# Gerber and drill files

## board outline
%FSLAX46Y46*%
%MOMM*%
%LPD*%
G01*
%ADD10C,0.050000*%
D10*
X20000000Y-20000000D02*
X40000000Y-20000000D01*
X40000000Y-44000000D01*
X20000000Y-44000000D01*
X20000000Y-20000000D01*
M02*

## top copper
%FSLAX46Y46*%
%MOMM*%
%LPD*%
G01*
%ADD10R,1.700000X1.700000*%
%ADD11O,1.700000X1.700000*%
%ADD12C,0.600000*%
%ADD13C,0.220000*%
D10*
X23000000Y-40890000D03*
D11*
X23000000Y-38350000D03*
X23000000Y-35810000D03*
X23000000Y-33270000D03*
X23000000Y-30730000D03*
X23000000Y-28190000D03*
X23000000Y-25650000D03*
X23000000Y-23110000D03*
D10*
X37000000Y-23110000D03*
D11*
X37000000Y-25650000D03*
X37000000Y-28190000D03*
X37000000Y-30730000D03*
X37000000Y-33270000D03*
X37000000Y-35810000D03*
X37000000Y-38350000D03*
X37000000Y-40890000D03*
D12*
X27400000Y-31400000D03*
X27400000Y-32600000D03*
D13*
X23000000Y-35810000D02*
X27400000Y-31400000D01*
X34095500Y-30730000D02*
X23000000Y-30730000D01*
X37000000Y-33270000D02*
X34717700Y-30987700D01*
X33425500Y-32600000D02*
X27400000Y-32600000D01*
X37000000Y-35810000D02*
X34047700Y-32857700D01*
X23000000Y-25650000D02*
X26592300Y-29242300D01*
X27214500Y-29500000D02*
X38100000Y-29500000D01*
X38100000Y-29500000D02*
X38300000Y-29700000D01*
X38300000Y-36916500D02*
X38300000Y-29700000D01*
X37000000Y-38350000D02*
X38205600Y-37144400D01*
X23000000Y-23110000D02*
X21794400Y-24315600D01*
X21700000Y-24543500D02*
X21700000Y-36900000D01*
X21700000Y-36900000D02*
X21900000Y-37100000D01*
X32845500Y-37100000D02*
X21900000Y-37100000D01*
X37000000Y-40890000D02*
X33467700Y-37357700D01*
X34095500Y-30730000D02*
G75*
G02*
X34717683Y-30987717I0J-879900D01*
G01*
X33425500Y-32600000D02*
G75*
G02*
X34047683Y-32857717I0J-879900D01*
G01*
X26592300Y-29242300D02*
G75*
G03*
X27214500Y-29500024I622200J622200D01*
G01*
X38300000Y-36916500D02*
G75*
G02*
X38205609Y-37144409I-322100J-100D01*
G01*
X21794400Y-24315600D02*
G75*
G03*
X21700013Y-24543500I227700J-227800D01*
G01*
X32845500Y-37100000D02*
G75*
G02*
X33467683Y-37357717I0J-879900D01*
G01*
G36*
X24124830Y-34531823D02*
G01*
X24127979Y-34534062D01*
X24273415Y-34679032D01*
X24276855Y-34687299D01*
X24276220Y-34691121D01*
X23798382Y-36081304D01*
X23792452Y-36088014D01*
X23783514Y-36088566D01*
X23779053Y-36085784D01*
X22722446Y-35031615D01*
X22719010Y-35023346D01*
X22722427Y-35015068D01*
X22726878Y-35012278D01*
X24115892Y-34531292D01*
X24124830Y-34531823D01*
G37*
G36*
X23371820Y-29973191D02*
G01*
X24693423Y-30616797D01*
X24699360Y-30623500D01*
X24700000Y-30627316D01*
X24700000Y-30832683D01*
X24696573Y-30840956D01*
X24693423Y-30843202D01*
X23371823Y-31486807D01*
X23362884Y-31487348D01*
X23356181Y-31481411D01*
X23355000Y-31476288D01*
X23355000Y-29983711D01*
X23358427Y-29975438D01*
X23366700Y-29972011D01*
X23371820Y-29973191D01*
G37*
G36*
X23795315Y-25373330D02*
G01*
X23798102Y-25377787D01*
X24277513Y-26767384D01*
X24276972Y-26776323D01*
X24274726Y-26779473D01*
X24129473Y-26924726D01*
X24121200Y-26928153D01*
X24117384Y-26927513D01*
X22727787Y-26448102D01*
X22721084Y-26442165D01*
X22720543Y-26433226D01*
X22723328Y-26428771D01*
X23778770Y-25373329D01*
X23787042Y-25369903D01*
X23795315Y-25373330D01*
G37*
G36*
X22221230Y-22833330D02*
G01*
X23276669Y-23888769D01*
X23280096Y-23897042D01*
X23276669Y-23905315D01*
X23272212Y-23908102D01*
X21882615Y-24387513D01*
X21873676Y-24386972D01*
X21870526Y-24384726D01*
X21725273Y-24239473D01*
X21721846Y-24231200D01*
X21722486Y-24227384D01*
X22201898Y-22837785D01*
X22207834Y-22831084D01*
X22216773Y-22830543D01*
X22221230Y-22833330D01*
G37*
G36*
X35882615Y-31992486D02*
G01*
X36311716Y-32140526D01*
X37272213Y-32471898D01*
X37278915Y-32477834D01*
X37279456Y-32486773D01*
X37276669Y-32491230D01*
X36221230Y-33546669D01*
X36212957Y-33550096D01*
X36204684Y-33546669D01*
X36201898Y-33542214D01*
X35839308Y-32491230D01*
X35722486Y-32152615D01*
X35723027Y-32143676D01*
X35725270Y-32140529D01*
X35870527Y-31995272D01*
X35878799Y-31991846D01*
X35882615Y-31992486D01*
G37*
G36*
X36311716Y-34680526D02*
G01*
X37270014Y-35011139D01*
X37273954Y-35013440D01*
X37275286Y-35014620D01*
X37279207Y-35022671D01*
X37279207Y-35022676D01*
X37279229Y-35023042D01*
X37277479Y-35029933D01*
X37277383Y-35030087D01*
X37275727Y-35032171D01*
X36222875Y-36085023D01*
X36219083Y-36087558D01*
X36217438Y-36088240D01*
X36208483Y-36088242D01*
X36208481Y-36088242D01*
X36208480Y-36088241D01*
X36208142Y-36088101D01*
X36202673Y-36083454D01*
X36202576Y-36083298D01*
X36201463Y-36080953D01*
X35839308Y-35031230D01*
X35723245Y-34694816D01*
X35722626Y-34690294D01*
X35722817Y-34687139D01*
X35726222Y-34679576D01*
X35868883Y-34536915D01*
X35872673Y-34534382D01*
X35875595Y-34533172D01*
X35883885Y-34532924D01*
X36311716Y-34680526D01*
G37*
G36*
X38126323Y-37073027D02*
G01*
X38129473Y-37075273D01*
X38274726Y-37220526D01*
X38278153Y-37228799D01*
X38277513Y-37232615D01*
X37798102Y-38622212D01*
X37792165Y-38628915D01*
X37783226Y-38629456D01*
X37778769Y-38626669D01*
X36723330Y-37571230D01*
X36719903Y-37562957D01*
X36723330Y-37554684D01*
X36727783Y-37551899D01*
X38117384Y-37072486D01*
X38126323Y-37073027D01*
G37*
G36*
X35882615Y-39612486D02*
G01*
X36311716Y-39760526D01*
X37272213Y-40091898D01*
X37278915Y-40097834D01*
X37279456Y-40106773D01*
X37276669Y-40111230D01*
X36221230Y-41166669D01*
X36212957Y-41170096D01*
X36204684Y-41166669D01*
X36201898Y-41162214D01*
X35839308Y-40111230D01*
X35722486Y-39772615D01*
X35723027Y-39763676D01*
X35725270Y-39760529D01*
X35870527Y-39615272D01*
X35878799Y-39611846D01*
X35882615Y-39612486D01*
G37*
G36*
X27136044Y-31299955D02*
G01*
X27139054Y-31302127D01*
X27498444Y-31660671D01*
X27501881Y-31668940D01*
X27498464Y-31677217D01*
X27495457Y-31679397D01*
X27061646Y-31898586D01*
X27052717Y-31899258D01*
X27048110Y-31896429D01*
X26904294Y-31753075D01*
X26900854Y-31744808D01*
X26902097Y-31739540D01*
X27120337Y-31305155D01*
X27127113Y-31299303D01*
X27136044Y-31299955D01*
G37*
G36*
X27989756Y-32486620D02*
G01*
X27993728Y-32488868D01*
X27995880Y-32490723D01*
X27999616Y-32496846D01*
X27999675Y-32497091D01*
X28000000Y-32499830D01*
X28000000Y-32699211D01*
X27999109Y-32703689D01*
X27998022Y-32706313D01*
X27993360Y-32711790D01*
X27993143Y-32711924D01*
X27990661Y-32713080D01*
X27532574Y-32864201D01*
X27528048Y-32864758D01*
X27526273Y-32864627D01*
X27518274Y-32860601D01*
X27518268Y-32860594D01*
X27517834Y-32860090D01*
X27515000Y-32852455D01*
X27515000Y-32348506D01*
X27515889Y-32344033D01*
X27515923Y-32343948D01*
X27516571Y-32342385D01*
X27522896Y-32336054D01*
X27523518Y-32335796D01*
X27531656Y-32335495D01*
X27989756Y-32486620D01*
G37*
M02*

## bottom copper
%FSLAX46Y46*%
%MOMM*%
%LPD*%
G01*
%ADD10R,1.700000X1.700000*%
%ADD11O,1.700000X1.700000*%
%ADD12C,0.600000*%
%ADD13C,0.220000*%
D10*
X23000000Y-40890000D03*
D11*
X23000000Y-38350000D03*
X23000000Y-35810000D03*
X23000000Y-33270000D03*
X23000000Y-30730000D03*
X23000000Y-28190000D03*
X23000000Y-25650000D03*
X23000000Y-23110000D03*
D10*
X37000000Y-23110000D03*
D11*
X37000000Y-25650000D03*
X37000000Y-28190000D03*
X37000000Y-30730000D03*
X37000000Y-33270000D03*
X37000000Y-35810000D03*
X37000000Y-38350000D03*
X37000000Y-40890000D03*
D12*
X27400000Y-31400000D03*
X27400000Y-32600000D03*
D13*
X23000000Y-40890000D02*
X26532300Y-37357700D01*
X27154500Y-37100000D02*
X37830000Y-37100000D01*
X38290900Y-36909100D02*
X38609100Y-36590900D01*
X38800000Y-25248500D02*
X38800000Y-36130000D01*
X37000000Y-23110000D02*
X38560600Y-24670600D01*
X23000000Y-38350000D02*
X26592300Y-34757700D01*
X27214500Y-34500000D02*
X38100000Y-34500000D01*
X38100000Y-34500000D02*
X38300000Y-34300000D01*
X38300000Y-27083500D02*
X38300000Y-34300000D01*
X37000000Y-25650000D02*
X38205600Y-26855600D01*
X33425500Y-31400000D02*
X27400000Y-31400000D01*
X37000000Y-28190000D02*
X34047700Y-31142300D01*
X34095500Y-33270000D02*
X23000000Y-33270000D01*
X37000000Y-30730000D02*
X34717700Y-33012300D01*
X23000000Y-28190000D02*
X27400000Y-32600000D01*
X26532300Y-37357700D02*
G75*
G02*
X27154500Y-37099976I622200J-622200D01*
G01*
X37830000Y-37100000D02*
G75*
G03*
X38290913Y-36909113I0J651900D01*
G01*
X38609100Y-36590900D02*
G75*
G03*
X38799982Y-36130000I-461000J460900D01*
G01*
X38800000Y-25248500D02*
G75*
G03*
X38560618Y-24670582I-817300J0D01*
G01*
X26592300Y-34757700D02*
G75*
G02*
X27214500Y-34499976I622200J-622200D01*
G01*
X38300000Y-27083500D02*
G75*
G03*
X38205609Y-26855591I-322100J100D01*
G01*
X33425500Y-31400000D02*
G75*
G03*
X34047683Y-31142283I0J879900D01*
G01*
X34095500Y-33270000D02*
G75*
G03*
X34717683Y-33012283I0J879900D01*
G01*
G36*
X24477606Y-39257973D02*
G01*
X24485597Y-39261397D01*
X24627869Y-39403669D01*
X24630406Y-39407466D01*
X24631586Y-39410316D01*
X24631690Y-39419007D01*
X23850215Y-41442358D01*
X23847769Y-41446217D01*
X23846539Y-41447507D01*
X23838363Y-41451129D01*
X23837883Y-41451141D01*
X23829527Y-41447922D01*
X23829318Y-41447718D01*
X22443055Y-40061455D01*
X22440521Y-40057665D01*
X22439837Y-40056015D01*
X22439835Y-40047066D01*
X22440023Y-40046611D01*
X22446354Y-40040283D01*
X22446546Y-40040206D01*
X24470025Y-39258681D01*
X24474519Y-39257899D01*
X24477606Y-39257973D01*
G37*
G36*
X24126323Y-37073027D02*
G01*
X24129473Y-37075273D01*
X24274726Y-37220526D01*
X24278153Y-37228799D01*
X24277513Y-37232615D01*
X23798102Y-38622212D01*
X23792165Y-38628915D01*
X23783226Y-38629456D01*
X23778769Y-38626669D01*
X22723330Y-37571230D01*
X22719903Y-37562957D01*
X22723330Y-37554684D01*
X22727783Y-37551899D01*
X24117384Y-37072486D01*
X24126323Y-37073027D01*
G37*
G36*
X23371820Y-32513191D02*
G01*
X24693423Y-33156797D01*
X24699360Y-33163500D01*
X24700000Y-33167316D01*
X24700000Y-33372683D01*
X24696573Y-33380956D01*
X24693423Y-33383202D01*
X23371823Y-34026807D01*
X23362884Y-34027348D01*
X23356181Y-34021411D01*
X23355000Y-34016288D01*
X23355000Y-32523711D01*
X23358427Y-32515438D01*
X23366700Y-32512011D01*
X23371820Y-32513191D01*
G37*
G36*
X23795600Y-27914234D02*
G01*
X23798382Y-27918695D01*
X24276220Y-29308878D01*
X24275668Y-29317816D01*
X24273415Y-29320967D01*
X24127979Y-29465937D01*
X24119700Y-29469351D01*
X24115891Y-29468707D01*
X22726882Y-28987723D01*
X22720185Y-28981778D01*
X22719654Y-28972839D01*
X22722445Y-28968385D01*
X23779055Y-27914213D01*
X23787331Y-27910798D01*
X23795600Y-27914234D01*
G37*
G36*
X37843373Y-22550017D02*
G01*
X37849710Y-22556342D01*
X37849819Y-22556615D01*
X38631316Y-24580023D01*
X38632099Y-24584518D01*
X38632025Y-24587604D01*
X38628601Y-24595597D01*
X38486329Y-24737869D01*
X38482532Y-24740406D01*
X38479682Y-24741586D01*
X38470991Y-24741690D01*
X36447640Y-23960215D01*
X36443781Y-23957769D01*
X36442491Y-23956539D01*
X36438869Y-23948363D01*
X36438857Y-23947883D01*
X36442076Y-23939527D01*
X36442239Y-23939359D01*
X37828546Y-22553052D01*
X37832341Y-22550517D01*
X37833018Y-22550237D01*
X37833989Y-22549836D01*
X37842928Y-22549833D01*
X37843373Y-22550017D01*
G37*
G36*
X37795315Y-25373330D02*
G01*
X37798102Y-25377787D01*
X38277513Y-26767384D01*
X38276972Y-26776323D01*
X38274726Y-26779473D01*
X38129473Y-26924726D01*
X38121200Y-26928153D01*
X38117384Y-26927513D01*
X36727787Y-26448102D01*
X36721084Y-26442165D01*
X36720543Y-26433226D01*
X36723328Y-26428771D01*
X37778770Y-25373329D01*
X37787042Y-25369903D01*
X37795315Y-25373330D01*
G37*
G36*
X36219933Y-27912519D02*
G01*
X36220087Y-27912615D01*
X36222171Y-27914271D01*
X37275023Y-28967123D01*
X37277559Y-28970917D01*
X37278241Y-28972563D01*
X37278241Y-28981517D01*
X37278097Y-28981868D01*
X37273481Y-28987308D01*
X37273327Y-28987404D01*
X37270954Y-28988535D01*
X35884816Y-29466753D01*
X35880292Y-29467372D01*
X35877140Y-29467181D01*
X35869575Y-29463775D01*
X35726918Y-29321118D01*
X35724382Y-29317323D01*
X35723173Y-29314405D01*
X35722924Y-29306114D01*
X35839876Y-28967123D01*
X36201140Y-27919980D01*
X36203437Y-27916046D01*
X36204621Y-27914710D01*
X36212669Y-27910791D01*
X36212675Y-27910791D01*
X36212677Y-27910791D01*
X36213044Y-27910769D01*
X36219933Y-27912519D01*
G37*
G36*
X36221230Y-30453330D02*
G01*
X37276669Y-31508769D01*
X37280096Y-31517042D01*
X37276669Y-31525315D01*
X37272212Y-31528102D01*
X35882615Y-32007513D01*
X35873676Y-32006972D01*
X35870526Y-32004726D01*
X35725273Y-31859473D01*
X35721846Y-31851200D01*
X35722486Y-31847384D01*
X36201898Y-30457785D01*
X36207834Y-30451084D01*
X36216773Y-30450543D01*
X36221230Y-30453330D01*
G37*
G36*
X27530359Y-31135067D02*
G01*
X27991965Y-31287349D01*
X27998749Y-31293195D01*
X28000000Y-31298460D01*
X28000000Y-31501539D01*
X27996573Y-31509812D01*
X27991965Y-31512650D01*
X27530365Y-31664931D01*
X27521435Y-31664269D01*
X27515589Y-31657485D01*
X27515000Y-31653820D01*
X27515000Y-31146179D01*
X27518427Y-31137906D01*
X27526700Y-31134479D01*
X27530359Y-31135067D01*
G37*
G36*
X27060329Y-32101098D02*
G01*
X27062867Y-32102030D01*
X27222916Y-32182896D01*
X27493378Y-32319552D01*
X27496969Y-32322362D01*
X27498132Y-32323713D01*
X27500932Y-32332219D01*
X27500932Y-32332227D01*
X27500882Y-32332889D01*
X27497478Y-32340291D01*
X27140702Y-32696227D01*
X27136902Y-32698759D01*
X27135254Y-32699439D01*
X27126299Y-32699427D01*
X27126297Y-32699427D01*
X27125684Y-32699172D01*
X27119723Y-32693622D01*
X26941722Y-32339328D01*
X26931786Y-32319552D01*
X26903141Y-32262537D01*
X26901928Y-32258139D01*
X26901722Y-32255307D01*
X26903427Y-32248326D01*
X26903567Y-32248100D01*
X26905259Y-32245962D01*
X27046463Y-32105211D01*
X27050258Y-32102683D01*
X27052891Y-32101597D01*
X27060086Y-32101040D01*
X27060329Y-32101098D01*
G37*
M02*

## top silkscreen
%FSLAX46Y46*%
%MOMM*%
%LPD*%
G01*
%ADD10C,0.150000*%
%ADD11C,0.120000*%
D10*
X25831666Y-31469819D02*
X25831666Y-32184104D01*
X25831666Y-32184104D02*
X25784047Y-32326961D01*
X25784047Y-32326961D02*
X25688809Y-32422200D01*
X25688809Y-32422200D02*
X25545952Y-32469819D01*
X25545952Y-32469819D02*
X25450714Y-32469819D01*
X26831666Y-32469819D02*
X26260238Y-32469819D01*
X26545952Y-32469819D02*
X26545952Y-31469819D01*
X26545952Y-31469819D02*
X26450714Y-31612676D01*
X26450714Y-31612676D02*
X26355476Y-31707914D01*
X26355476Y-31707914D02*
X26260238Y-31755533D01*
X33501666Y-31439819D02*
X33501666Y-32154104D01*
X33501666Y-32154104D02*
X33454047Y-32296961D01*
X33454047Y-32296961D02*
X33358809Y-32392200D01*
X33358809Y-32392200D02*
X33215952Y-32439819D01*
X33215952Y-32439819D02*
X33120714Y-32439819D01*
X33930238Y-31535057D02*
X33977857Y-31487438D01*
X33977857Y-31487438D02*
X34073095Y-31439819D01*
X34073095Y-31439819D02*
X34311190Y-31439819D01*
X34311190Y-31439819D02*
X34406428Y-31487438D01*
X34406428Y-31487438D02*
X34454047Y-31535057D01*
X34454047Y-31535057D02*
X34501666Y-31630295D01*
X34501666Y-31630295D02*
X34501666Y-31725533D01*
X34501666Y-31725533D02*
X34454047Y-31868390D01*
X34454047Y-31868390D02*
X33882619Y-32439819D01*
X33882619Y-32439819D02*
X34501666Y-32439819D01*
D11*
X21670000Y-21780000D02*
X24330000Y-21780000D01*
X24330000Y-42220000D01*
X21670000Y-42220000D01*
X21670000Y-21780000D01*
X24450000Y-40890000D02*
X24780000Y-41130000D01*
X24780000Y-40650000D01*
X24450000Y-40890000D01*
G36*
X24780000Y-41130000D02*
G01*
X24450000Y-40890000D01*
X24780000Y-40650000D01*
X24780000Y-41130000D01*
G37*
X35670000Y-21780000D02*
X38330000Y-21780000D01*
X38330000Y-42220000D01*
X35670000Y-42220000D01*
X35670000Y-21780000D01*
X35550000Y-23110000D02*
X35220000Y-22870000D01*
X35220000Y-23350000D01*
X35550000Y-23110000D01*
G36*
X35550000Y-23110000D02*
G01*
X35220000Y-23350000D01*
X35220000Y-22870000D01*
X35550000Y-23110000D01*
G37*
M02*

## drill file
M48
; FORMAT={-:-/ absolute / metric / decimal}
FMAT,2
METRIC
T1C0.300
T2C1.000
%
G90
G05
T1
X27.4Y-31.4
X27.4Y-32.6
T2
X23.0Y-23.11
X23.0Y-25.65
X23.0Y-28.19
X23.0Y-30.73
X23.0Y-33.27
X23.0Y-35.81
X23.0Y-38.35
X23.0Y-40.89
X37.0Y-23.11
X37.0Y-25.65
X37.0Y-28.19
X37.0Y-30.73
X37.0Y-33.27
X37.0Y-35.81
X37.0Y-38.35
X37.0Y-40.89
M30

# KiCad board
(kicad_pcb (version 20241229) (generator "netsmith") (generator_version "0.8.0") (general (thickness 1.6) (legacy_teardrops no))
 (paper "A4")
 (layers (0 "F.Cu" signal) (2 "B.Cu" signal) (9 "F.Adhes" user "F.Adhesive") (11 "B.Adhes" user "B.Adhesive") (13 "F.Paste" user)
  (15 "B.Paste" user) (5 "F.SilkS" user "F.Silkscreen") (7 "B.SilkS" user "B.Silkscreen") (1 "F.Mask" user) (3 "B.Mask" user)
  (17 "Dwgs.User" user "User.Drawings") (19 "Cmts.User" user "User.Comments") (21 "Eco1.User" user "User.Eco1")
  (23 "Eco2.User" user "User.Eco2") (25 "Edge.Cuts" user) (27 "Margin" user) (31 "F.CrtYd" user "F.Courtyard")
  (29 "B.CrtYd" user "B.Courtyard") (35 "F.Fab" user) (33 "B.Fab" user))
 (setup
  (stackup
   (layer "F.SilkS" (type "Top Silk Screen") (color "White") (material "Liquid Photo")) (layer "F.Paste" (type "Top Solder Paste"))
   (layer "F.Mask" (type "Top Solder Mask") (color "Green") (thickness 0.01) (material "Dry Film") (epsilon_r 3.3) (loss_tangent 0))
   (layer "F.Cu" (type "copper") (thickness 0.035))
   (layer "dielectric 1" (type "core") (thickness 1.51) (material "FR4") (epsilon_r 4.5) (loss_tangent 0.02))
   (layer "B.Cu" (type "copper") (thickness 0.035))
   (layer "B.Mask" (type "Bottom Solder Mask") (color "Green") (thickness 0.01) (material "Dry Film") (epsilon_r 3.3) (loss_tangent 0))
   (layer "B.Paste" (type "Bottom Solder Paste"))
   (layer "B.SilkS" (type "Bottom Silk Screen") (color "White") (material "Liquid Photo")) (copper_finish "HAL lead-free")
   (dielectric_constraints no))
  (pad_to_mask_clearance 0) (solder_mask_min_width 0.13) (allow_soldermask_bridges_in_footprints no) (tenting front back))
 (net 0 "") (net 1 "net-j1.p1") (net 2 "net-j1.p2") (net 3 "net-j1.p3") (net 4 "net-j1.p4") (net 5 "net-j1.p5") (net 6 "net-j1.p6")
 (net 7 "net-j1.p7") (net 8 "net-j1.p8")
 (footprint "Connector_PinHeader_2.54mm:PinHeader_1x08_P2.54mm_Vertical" (layer "F.Cu") (at 23 40.89 180)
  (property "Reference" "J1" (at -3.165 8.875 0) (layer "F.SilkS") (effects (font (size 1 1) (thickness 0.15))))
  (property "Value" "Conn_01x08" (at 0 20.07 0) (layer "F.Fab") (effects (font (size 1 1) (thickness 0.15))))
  (pad "1" thru_hole rect (at 0 0 180) (size 1.7 1.7) (drill 1) (layers "*.Cu" "*.Mask") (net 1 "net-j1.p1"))
  (pad "2" thru_hole oval (at 0 2.54 180) (size 1.7 1.7) (drill 1) (layers "*.Cu" "*.Mask") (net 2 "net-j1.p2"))
  (pad "3" thru_hole oval (at 0 5.08 180) (size 1.7 1.7) (drill 1) (layers "*.Cu" "*.Mask") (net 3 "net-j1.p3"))
  (pad "4" thru_hole oval (at 0 7.62 180) (size 1.7 1.7) (drill 1) (layers "*.Cu" "*.Mask") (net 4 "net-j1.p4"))
  (pad "5" thru_hole oval (at 0 10.16 180) (size 1.7 1.7) (drill 1) (layers "*.Cu" "*.Mask") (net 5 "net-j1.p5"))
  (pad "6" thru_hole oval (at 0 12.7 180) (size 1.7 1.7) (drill 1) (layers "*.Cu" "*.Mask") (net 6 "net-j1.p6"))
  (pad "7" thru_hole oval (at 0 15.24 180) (size 1.7 1.7) (drill 1) (layers "*.Cu" "*.Mask") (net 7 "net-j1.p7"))
  (pad "8" thru_hole oval (at 0 17.78 180) (size 1.7 1.7) (drill 1) (layers "*.Cu" "*.Mask") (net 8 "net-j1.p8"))
  (fp_rect (start -1.33 -1.33) (end 1.33 19.11) (stroke (width 0.12) (type solid)) (fill no) (layer "F.SilkS"))
  (fp_poly (pts (xy -1.45 0) (xy -1.78 -0.24) (xy -1.78 0.24)) (stroke (width 0.12) (type solid)) (fill solid) (layer "F.SilkS")))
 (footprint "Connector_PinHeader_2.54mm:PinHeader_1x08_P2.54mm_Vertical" (layer "F.Cu") (at 37 23.11)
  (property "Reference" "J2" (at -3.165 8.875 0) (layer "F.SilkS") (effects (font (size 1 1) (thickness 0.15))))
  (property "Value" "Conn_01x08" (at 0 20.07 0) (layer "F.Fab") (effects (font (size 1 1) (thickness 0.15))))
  (pad "1" thru_hole rect (at 0 0) (size 1.7 1.7) (drill 1) (layers "*.Cu" "*.Mask") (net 1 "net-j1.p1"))
  (pad "2" thru_hole oval (at 0 2.54) (size 1.7 1.7) (drill 1) (layers "*.Cu" "*.Mask") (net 2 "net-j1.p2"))
  (pad "3" thru_hole oval (at 0 5.08) (size 1.7 1.7) (drill 1) (layers "*.Cu" "*.Mask") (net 3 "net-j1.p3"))
  (pad "4" thru_hole oval (at 0 7.62) (size 1.7 1.7) (drill 1) (layers "*.Cu" "*.Mask") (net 4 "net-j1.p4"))
  (pad "5" thru_hole oval (at 0 10.16) (size 1.7 1.7) (drill 1) (layers "*.Cu" "*.Mask") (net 5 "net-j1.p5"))
  (pad "6" thru_hole oval (at 0 12.7) (size 1.7 1.7) (drill 1) (layers "*.Cu" "*.Mask") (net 6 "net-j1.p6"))
  (pad "7" thru_hole oval (at 0 15.24) (size 1.7 1.7) (drill 1) (layers "*.Cu" "*.Mask") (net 7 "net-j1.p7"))
  (pad "8" thru_hole oval (at 0 17.78) (size 1.7 1.7) (drill 1) (layers "*.Cu" "*.Mask") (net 8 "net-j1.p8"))
  (fp_rect (start -1.33 -1.33) (end 1.33 19.11) (stroke (width 0.12) (type solid)) (fill no) (layer "F.SilkS"))
  (fp_poly (pts (xy -1.45 0) (xy -1.78 -0.24) (xy -1.78 0.24)) (stroke (width 0.12) (type solid)) (fill solid) (layer "F.SilkS")))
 (segment (start 23 40.89) (end 26.5323 37.3577) (width 0.22) (layer "B.Cu") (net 1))
 (segment (start 27.1545 37.1) (end 37.83 37.1) (width 0.22) (layer "B.Cu") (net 1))
 (segment (start 38.2909 36.9091) (end 38.6091 36.5909) (width 0.22) (layer "B.Cu") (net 1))
 (segment (start 38.8 25.2485) (end 38.8 36.13) (width 0.22) (layer "B.Cu") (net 1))
 (segment (start 37 23.11) (end 38.5606 24.6706) (width 0.22) (layer "B.Cu") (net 1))
 (segment (start 23 38.35) (end 26.5923 34.7577) (width 0.22) (layer "B.Cu") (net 2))
 (segment (start 27.2145 34.5) (end 38.1 34.5) (width 0.22) (layer "B.Cu") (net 2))
 (segment (start 38.1 34.5) (end 38.3 34.3) (width 0.22) (layer "B.Cu") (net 2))
 (segment (start 38.3 27.0835) (end 38.3 34.3) (width 0.22) (layer "B.Cu") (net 2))
 (segment (start 37 25.65) (end 38.2056 26.8556) (width 0.22) (layer "B.Cu") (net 2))
 (segment (start 23 35.81) (end 27.4 31.4) (width 0.22) (layer "F.Cu") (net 3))
 (segment (start 33.4255 31.4) (end 27.4 31.4) (width 0.22) (layer "B.Cu") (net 3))
 (segment (start 37 28.19) (end 34.0477 31.1423) (width 0.22) (layer "B.Cu") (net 3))
 (segment (start 34.0955 33.27) (end 23 33.27) (width 0.22) (layer "B.Cu") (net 4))
 (segment (start 37 30.73) (end 34.7177 33.0123) (width 0.22) (layer "B.Cu") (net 4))
 (segment (start 34.0955 30.73) (end 23 30.73) (width 0.22) (layer "F.Cu") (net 5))
 (segment (start 37 33.27) (end 34.7177 30.9877) (width 0.22) (layer "F.Cu") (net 5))
 (segment (start 23 28.19) (end 27.4 32.6) (width 0.22) (layer "B.Cu") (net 6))
 (segment (start 33.4255 32.6) (end 27.4 32.6) (width 0.22) (layer "F.Cu") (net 6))
 (segment (start 37 35.81) (end 34.0477 32.8577) (width 0.22) (layer "F.Cu") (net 6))
 (segment (start 23 25.65) (end 26.5923 29.2423) (width 0.22) (layer "F.Cu") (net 7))
 (segment (start 27.2145 29.5) (end 38.1 29.5) (width 0.22) (layer "F.Cu") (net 7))
 (segment (start 38.1 29.5) (end 38.3 29.7) (width 0.22) (layer "F.Cu") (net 7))
 (segment (start 38.3 36.9165) (end 38.3 29.7) (width 0.22) (layer "F.Cu") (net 7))
 (segment (start 37 38.35) (end 38.2056 37.1444) (width 0.22) (layer "F.Cu") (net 7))
 (segment (start 23 23.11) (end 21.7944 24.3156) (width 0.22) (layer "F.Cu") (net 8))
 (segment (start 21.7 24.5435) (end 21.7 36.9) (width 0.22) (layer "F.Cu") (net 8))
 (segment (start 21.7 36.9) (end 21.9 37.1) (width 0.22) (layer "F.Cu") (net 8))
 (segment (start 32.8455 37.1) (end 21.9 37.1) (width 0.22) (layer "F.Cu") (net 8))
 (segment (start 37 40.89) (end 33.4677 37.3577) (width 0.22) (layer "F.Cu") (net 8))
 (arc (start 26.5323 37.3577) (mid 26.8177 37.167) (end 27.1545 37.1) (width 0.22) (layer "B.Cu") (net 1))
 (arc (start 37.83 37.1) (mid 38.0794 37.0504) (end 38.2909 36.9091) (width 0.22) (layer "B.Cu") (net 1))
 (arc (start 38.6091 36.5909) (mid 38.7504 36.3794) (end 38.8 36.13) (width 0.22) (layer "B.Cu") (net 1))
 (arc (start 38.8 25.2485) (mid 38.7378 24.9358) (end 38.5606 24.6706) (width 0.22) (layer "B.Cu") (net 1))
 (arc (start 26.5923 34.7577) (mid 26.8777 34.567) (end 27.2145 34.5) (width 0.22) (layer "B.Cu") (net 2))
 (arc (start 38.3 27.0835) (mid 38.2755 26.9602) (end 38.2056 26.8556) (width 0.22) (layer "B.Cu") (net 2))
 (arc (start 33.4255 31.4) (mid 33.7623 31.333) (end 34.0477 31.1423) (width 0.22) (layer "B.Cu") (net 3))
 (arc (start 34.0955 33.27) (mid 34.4323 33.203) (end 34.7177 33.0123) (width 0.22) (layer "B.Cu") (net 4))
 (arc (start 34.0955 30.73) (mid 34.4323 30.797) (end 34.7177 30.9877) (width 0.22) (layer "F.Cu") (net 5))
 (arc (start 33.4255 32.6) (mid 33.7623 32.667) (end 34.0477 32.8577) (width 0.22) (layer "F.Cu") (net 6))
 (arc (start 26.5923 29.2423) (mid 26.8777 29.433) (end 27.2145 29.5) (width 0.22) (layer "F.Cu") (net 7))
 (arc (start 38.3 36.9165) (mid 38.2755 37.0398) (end 38.2056 37.1444) (width 0.22) (layer "F.Cu") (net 7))
 (arc (start 21.7944 24.3156) (mid 21.7245 24.4202) (end 21.7 24.5435) (width 0.22) (layer "F.Cu") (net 8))
 (arc (start 32.8455 37.1) (mid 33.1823 37.167) (end 33.4677 37.3577) (width 0.22) (layer "F.Cu") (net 8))
 (via (at 27.4 31.4) (size 0.6) (drill 0.3) (layers "F.Cu" "B.Cu") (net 3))
 (via (at 27.4 32.6) (size 0.6) (drill 0.3) (layers "F.Cu" "B.Cu") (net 6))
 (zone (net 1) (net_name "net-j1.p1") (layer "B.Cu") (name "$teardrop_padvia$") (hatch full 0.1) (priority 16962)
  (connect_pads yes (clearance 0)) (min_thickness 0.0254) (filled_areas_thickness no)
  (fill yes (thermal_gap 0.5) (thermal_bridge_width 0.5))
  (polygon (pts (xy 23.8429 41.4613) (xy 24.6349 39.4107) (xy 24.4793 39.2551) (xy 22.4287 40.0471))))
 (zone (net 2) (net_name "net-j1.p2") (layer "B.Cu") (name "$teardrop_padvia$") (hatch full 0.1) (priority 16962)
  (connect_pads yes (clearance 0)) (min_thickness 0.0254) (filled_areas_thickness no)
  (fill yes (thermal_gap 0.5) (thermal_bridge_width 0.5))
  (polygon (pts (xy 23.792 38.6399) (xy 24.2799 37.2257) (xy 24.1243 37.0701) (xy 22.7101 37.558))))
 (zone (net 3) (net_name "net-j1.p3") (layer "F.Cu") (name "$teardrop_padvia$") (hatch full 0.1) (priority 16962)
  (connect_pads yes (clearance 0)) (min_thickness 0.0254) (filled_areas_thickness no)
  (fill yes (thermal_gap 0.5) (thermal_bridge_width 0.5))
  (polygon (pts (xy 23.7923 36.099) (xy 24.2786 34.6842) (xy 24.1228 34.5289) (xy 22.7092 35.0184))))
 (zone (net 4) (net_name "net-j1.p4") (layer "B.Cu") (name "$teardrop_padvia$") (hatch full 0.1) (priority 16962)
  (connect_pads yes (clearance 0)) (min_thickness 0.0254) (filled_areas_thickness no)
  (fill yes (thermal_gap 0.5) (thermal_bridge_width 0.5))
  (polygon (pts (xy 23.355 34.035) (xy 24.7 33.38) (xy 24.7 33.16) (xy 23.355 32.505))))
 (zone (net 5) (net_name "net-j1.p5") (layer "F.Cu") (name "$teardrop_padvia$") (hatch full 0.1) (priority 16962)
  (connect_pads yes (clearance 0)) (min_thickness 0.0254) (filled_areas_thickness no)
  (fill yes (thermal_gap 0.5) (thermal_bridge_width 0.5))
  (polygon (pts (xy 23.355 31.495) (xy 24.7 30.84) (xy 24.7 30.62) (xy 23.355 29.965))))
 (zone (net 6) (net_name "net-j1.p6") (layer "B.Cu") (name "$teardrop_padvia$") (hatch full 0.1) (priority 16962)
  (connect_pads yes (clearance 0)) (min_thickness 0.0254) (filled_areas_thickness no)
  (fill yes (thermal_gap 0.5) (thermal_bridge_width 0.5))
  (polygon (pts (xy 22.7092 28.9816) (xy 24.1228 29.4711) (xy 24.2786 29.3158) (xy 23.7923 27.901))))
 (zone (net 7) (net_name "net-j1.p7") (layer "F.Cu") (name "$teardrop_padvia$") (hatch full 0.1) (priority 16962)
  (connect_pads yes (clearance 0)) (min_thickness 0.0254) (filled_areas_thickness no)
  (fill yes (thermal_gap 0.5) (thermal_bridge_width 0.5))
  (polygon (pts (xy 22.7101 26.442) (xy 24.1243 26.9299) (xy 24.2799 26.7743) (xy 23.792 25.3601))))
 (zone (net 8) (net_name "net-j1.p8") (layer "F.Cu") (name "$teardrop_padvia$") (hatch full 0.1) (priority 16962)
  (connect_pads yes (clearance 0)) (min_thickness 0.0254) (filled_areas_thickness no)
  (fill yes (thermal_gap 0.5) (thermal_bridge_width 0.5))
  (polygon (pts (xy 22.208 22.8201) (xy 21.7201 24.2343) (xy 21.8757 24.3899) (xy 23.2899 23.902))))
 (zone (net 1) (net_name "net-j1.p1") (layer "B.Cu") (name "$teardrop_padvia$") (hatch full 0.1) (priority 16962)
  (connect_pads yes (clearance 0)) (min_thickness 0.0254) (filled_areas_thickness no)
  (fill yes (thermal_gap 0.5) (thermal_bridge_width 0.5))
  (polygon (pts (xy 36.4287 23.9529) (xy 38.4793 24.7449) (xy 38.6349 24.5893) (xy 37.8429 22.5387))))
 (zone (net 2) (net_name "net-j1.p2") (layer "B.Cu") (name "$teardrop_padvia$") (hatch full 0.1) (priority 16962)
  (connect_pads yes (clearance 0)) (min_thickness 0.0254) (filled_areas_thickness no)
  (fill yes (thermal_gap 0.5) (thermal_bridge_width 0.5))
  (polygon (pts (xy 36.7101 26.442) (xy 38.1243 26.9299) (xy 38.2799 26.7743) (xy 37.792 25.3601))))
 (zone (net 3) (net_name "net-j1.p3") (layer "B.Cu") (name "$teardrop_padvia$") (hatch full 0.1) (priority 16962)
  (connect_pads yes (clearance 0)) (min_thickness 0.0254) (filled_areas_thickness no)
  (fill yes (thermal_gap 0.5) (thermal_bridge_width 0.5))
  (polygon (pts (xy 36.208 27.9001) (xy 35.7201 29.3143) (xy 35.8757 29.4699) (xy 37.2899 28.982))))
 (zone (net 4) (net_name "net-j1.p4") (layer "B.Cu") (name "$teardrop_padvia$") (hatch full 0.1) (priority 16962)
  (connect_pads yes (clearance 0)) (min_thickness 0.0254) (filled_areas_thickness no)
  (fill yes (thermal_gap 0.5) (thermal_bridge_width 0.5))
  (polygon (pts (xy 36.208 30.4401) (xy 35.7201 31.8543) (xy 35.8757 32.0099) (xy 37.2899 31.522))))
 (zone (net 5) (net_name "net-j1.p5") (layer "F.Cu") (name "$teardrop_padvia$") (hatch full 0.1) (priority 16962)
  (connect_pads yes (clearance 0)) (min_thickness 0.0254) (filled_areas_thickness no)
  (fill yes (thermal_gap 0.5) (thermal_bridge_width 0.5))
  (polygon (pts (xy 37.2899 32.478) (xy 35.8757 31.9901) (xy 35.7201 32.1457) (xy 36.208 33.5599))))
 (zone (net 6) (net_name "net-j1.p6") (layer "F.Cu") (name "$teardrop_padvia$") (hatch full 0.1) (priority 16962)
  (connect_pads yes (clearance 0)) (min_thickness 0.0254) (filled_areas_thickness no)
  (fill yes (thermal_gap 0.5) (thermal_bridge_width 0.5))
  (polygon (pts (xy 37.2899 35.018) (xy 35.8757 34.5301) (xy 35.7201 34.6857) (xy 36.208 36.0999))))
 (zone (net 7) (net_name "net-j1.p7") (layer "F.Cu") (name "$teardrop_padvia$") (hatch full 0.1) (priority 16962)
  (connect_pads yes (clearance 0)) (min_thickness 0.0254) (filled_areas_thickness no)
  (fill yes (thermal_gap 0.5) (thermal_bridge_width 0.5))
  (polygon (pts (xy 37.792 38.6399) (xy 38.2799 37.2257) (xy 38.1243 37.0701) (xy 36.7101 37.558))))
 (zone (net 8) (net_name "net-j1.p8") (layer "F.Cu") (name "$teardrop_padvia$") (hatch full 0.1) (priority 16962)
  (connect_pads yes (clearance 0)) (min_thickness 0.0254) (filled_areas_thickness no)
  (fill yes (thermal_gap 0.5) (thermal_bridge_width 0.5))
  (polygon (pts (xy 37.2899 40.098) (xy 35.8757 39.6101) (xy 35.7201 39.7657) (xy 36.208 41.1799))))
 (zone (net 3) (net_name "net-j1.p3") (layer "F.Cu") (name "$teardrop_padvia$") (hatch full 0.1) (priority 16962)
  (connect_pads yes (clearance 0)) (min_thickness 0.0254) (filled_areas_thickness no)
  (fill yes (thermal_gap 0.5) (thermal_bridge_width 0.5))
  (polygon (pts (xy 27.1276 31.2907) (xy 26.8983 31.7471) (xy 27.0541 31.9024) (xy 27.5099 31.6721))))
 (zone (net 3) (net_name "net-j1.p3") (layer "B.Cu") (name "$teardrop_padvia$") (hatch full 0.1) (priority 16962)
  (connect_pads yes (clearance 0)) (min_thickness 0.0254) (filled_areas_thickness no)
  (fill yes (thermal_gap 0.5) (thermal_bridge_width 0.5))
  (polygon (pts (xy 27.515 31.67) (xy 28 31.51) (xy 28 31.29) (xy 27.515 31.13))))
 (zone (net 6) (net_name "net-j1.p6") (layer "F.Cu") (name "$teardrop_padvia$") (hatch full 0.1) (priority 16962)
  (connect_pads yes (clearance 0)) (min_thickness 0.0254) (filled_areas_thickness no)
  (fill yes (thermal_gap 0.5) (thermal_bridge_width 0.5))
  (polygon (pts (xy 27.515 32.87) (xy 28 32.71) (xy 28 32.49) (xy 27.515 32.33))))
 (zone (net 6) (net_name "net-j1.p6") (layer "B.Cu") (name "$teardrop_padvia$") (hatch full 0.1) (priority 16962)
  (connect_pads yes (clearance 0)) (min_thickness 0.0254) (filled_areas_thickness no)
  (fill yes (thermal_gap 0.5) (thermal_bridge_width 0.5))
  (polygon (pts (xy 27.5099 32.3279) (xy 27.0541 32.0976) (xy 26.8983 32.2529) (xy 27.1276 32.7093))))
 (gr_rect (start 20 20) (end 40 44) (stroke (width 0.05) (type default)) (fill no) (layer "Edge.Cuts")))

